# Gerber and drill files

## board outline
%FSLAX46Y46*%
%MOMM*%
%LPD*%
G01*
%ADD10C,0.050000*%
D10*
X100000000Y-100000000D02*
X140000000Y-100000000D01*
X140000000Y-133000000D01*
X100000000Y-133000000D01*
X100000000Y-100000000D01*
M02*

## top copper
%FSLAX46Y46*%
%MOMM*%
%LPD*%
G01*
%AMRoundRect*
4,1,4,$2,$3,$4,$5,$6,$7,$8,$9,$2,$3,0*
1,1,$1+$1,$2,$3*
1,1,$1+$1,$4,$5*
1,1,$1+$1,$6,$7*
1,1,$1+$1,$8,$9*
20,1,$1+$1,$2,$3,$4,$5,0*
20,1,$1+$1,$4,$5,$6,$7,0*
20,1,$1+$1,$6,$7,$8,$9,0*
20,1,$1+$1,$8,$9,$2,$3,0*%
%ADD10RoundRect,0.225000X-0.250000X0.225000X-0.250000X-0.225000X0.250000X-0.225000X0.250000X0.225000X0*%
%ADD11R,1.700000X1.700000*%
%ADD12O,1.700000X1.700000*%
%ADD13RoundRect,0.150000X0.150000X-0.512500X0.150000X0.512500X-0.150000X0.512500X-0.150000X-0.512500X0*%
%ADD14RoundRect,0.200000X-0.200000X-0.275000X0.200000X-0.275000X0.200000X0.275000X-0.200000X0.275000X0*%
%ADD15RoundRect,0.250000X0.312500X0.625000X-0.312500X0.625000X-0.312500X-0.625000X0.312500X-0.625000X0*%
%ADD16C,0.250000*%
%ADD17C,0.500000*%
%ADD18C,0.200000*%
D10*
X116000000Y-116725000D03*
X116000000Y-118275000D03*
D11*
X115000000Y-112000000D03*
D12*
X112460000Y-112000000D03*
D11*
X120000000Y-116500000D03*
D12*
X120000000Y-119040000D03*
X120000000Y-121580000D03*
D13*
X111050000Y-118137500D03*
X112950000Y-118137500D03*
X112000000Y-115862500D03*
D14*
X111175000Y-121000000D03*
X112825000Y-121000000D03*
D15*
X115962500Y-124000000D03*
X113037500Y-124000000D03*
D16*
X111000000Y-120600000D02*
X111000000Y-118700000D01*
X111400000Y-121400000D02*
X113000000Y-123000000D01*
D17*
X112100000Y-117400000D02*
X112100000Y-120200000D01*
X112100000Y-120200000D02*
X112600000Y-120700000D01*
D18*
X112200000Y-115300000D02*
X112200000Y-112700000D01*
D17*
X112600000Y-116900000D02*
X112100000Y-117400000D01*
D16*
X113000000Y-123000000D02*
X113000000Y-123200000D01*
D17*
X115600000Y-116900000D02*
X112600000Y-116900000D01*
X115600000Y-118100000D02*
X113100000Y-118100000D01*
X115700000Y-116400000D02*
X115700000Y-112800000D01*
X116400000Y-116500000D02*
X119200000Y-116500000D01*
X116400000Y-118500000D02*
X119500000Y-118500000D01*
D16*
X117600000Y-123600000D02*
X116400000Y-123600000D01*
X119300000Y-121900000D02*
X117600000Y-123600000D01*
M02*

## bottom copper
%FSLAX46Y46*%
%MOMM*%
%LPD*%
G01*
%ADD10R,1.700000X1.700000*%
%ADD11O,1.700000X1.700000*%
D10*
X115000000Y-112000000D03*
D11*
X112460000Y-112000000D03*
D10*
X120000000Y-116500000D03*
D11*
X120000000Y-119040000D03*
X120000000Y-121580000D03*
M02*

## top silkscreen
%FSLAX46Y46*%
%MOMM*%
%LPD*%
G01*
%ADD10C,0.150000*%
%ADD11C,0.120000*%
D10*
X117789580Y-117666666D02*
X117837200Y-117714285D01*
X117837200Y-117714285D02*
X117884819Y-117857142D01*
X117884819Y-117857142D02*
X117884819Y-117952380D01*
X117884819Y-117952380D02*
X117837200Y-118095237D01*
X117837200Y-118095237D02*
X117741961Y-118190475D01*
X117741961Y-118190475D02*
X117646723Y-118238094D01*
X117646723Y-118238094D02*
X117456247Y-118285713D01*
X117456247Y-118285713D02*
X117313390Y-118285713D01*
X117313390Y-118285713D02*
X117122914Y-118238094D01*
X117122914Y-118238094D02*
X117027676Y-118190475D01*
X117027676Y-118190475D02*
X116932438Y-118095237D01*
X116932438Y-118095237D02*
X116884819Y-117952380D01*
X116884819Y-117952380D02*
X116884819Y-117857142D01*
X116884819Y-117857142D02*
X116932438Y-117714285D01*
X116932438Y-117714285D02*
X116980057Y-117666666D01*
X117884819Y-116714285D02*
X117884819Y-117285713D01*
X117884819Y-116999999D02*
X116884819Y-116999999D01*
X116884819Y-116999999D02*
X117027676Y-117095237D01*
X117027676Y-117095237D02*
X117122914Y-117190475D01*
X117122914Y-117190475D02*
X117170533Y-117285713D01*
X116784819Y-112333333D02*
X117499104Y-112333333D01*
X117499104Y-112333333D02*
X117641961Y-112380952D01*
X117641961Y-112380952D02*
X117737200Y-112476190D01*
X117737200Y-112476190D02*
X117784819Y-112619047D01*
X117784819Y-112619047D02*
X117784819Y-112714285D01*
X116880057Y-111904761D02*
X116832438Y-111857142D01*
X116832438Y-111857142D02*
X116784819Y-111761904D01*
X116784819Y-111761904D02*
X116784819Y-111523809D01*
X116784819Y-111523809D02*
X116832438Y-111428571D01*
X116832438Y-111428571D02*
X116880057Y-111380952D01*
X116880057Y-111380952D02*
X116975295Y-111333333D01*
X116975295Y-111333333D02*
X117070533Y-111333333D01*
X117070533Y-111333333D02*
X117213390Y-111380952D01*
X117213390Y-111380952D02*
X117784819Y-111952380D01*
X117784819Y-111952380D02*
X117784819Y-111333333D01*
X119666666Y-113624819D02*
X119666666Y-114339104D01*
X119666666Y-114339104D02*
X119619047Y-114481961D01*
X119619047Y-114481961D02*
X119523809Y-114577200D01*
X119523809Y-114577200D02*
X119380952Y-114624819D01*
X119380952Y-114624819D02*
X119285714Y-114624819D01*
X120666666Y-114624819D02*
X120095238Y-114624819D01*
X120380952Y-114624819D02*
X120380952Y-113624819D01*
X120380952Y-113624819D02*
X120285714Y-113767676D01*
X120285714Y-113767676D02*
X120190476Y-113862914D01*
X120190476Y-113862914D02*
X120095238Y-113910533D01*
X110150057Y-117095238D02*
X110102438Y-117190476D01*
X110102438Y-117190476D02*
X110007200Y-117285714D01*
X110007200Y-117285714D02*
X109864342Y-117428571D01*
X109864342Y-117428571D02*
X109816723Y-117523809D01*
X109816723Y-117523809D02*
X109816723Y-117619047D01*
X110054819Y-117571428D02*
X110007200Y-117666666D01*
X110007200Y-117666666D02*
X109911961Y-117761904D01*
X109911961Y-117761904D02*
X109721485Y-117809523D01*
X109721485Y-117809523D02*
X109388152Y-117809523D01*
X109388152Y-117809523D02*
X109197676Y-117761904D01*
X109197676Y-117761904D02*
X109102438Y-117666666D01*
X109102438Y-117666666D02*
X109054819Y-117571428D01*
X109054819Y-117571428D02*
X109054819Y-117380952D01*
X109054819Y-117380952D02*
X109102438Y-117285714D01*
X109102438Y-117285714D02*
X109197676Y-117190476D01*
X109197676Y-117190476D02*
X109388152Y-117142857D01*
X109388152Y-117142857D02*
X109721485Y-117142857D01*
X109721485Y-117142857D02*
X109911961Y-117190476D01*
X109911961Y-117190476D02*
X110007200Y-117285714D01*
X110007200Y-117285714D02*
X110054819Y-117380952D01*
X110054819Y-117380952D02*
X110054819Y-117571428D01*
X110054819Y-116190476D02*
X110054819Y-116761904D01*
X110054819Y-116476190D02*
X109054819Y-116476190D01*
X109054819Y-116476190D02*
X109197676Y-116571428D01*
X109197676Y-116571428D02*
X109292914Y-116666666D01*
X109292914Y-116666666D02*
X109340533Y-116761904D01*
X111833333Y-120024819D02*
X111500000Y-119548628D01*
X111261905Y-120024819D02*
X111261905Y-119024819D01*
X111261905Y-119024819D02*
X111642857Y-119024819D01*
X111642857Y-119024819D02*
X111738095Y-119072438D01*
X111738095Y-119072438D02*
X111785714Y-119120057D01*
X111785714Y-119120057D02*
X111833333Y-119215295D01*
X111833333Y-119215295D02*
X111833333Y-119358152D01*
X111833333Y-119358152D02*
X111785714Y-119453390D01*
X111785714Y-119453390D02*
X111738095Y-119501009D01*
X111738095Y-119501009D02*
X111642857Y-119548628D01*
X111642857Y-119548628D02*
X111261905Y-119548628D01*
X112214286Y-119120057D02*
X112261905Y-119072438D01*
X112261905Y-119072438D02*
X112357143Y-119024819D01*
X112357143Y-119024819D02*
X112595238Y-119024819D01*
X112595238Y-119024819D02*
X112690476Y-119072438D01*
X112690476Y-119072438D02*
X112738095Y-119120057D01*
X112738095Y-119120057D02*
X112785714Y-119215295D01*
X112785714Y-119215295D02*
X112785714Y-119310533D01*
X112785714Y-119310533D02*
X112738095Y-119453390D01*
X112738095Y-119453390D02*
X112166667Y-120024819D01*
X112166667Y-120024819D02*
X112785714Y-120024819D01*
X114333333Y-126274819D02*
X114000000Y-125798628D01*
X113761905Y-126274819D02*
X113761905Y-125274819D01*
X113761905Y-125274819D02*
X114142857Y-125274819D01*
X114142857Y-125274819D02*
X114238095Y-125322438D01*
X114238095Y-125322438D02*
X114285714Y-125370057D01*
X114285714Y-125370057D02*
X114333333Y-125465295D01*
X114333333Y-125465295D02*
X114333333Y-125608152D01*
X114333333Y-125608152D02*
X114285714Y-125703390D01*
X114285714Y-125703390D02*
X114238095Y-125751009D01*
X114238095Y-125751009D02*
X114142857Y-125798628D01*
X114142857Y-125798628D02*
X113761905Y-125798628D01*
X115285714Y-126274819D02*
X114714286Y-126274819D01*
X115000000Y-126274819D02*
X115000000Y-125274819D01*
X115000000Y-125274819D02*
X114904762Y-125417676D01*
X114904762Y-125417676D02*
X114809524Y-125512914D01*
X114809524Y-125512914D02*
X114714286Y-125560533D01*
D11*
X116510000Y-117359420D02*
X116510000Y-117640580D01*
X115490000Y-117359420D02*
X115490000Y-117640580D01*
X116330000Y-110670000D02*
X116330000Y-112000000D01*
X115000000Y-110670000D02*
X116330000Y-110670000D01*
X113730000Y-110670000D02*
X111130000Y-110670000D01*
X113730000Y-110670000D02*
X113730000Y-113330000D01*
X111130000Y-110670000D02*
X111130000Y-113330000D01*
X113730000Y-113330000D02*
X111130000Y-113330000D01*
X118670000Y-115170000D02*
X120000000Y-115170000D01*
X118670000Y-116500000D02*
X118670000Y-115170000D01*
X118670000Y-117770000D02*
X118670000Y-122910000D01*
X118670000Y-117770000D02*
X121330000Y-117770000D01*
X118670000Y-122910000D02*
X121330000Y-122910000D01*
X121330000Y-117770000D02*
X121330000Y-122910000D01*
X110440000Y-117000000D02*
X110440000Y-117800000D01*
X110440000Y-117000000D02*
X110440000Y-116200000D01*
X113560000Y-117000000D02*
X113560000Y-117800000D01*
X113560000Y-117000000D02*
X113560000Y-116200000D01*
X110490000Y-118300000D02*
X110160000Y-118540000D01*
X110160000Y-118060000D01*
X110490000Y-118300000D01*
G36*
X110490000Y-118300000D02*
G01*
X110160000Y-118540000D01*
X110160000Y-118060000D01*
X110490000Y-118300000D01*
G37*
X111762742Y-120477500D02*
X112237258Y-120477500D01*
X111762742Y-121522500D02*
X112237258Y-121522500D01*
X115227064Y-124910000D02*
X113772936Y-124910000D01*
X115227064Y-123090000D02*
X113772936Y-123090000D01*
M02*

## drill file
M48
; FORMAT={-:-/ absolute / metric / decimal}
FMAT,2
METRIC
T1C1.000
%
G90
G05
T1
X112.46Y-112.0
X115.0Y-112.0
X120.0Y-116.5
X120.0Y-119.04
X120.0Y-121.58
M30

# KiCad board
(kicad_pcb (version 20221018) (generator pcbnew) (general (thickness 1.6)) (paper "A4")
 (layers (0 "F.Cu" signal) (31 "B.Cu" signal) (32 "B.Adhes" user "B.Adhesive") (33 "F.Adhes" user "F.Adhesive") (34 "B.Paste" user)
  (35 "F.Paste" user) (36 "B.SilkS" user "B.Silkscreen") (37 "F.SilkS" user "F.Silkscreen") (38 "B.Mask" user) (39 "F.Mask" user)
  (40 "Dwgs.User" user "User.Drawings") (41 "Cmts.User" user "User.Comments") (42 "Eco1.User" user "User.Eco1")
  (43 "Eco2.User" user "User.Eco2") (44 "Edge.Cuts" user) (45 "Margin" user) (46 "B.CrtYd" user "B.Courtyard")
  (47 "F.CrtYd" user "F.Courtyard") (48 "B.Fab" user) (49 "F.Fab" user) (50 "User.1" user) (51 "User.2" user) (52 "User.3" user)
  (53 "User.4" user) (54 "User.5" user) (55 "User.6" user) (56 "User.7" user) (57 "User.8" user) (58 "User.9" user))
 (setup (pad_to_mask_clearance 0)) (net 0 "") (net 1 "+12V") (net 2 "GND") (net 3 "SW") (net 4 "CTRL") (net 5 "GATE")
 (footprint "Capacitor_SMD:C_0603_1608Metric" (layer "F.Cu") (at 116 117.5 -90)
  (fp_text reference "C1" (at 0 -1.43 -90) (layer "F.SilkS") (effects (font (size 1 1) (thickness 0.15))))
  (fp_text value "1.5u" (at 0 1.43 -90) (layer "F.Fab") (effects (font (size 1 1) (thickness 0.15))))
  (fp_line (start -0.14058 -0.51) (end 0.14058 -0.51) (stroke (width 0.12) (type solid)) (layer "F.SilkS"))
  (fp_line (start -0.14058 0.51) (end 0.14058 0.51) (stroke (width 0.12) (type solid)) (layer "F.SilkS"))
  (pad "1" smd roundrect (at -0.775 0 270) (size 0.9 0.95) (layers "F.Cu" "F.Paste" "F.Mask") (roundrect_rratio 0.25) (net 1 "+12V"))
  (pad "2" smd roundrect (at 0.775 0 270) (size 0.9 0.95) (layers "F.Cu" "F.Paste" "F.Mask") (roundrect_rratio 0.25) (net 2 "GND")))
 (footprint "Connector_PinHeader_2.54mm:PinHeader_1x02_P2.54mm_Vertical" (layer "F.Cu") (at 115 112 -90)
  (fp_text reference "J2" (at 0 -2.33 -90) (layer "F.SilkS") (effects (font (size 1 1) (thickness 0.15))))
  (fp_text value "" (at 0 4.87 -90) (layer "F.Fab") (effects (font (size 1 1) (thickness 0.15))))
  (fp_line (start -1.33 -1.33) (end 0 -1.33) (stroke (width 0.12) (type solid)) (layer "F.SilkS"))
  (fp_line (start -1.33 0) (end -1.33 -1.33) (stroke (width 0.12) (type solid)) (layer "F.SilkS"))
  (fp_line (start -1.33 1.27) (end -1.33 3.87) (stroke (width 0.12) (type solid)) (layer "F.SilkS"))
  (fp_line (start -1.33 1.27) (end 1.33 1.27) (stroke (width 0.12) (type solid)) (layer "F.SilkS"))
  (fp_line (start -1.33 3.87) (end 1.33 3.87) (stroke (width 0.12) (type solid)) (layer "F.SilkS"))
  (fp_line (start 1.33 1.27) (end 1.33 3.87) (stroke (width 0.12) (type solid)) (layer "F.SilkS"))
  (pad "1" thru_hole rect (at 0 0 270) (size 1.7 1.7) (drill 1) (layers "*.Cu" "*.Mask") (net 1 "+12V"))
  (pad "2" thru_hole oval (at 0 2.54 270) (size 1.7 1.7) (drill 1) (layers "*.Cu" "*.Mask") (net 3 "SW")))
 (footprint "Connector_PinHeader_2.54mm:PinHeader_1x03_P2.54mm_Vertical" (layer "F.Cu") (at 120 116.5)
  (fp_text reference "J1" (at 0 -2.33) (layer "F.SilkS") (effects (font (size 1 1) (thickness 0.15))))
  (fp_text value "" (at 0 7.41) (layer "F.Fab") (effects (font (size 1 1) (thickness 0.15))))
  (fp_line (start -1.33 -1.33) (end 0 -1.33) (stroke (width 0.12) (type solid)) (layer "F.SilkS"))
  (fp_line (start -1.33 0) (end -1.33 -1.33) (stroke (width 0.12) (type solid)) (layer "F.SilkS"))
  (fp_line (start -1.33 1.27) (end -1.33 6.41) (stroke (width 0.12) (type solid)) (layer "F.SilkS"))
  (fp_line (start -1.33 1.27) (end 1.33 1.27) (stroke (width 0.12) (type solid)) (layer "F.SilkS"))
  (fp_line (start -1.33 6.41) (end 1.33 6.41) (stroke (width 0.12) (type solid)) (layer "F.SilkS"))
  (fp_line (start 1.33 1.27) (end 1.33 6.41) (stroke (width 0.12) (type solid)) (layer "F.SilkS"))
  (pad "1" thru_hole rect (at 0 0) (size 1.7 1.7) (drill 1) (layers "*.Cu" "*.Mask") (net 1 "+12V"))
  (pad "2" thru_hole oval (at 0 2.54) (size 1.7 1.7) (drill 1) (layers "*.Cu" "*.Mask") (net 2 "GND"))
  (pad "3" thru_hole oval (at 0 5.08) (size 1.7 1.7) (drill 1) (layers "*.Cu" "*.Mask") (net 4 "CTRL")))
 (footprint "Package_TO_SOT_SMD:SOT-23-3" (layer "F.Cu") (at 112 117 90)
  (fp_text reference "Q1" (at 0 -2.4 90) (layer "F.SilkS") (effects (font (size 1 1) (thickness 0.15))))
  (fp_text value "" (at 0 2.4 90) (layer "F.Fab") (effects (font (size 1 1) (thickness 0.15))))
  (fp_line (start 0 -1.56) (end -0.8 -1.56) (stroke (width 0.12) (type solid)) (layer "F.SilkS"))
  (fp_line (start 0 -1.56) (end 0.8 -1.56) (stroke (width 0.12) (type solid)) (layer "F.SilkS"))
  (fp_line (start 0 1.56) (end -0.8 1.56) (stroke (width 0.12) (type solid)) (layer "F.SilkS"))
  (fp_line (start 0 1.56) (end 0.8 1.56) (stroke (width 0.12) (type solid)) (layer "F.SilkS"))
  (fp_poly
   (pts (xy -1.3 -1.51) (xy -1.54 -1.84) (xy -1.06 -1.84) (xy -1.3 -1.51)) (stroke (width 0.12) (type solid)) (fill solid) (layer "F.SilkS"))
  (pad "1" smd roundrect (at -1.1375 -0.95 90) (size 1.325 0.6) (layers "F.Cu" "F.Paste" "F.Mask") (roundrect_rratio 0.25) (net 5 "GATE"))
  (pad "2" smd roundrect (at -1.1375 0.95 90) (size 1.325 0.6) (layers "F.Cu" "F.Paste" "F.Mask") (roundrect_rratio 0.25) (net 2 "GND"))
  (pad "3" smd roundrect (at 1.1375 0 90) (size 1.325 0.6) (layers "F.Cu" "F.Paste" "F.Mask") (roundrect_rratio 0.25) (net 3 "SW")))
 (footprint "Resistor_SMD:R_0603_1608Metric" (layer "F.Cu") (at 112 121)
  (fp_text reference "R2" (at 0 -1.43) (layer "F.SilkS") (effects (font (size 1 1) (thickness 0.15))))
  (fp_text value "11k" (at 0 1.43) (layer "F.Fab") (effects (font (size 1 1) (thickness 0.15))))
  (fp_line (start -0.237258 -0.5225) (end 0.237258 -0.5225) (stroke (width 0.12) (type solid)) (layer "F.SilkS"))
  (fp_line (start -0.237258 0.5225) (end 0.237258 0.5225) (stroke (width 0.12) (type solid)) (layer "F.SilkS"))
  (pad "1" smd roundrect (at -0.825 0) (size 0.8 0.95) (layers "F.Cu" "F.Paste" "F.Mask") (roundrect_rratio 0.25) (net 5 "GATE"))
  (pad "2" smd roundrect (at 0.825 0) (size 0.8 0.95) (layers "F.Cu" "F.Paste" "F.Mask") (roundrect_rratio 0.25) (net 1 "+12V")))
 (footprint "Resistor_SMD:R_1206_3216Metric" (layer "F.Cu") (at 114.5 124 180)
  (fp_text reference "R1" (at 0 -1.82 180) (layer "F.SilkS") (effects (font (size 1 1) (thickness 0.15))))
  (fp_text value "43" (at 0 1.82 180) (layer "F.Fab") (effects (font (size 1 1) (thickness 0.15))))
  (fp_line (start -0.727064 -0.91) (end 0.727064 -0.91) (stroke (width 0.12) (type solid)) (layer "F.SilkS"))
  (fp_line (start -0.727064 0.91) (end 0.727064 0.91) (stroke (width 0.12) (type solid)) (layer "F.SilkS"))
  (pad "1" smd roundrect (at -1.4625 0 180) (size 1.125 1.75) (layers "F.Cu" "F.Paste" "F.Mask") (roundrect_rratio 0.222222) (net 4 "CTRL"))
  (pad "2" smd roundrect (at 1.4625 0 180) (size 1.125 1.75) (layers "F.Cu" "F.Paste" "F.Mask") (roundrect_rratio 0.222222) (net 5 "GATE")))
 (gr_rect (start 100 100) (end 140 133) (stroke (width 0.05) (type default)) (fill none) (layer "Edge.Cuts"))
 (segment (start 111 120.6) (end 111 118.7) (width 0.25) (layer "F.Cu") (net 5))
 (segment (start 111.4 121.4) (end 113 123) (width 0.25) (layer "F.Cu") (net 5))
 (segment (start 112.1 117.4) (end 112.1 120.2) (width 0.5) (layer "F.Cu") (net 1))
 (segment (start 112.1 120.2) (end 112.6 120.7) (width 0.5) (layer "F.Cu") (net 1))
 (segment (start 112.2 115.3) (end 112.2 112.7) (width 0.2) (layer "F.Cu") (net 3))
 (segment (start 112.6 116.9) (end 112.1 117.4) (width 0.5) (layer "F.Cu") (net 1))
 (segment (start 113 123) (end 113 123.2) (width 0.25) (layer "F.Cu") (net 5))
 (segment (start 115.6 116.9) (end 112.6 116.9) (width 0.5) (layer "F.Cu") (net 1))
 (segment (start 115.6 118.1) (end 113.1 118.1) (width 0.5) (layer "F.Cu") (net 2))
 (segment (start 115.7 116.4) (end 115.7 112.8) (width 0.5) (layer "F.Cu") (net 1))
 (segment (start 116.4 116.5) (end 119.2 116.5) (width 0.5) (layer "F.Cu") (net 1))
 (segment (start 116.4 118.5) (end 119.5 118.5) (width 0.5) (layer "F.Cu") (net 2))
 (segment (start 117.6 123.6) (end 116.4 123.6) (width 0.25) (layer "F.Cu") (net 4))
 (segment (start 119.3 121.9) (end 117.6 123.6) (width 0.25) (layer "F.Cu") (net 4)))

